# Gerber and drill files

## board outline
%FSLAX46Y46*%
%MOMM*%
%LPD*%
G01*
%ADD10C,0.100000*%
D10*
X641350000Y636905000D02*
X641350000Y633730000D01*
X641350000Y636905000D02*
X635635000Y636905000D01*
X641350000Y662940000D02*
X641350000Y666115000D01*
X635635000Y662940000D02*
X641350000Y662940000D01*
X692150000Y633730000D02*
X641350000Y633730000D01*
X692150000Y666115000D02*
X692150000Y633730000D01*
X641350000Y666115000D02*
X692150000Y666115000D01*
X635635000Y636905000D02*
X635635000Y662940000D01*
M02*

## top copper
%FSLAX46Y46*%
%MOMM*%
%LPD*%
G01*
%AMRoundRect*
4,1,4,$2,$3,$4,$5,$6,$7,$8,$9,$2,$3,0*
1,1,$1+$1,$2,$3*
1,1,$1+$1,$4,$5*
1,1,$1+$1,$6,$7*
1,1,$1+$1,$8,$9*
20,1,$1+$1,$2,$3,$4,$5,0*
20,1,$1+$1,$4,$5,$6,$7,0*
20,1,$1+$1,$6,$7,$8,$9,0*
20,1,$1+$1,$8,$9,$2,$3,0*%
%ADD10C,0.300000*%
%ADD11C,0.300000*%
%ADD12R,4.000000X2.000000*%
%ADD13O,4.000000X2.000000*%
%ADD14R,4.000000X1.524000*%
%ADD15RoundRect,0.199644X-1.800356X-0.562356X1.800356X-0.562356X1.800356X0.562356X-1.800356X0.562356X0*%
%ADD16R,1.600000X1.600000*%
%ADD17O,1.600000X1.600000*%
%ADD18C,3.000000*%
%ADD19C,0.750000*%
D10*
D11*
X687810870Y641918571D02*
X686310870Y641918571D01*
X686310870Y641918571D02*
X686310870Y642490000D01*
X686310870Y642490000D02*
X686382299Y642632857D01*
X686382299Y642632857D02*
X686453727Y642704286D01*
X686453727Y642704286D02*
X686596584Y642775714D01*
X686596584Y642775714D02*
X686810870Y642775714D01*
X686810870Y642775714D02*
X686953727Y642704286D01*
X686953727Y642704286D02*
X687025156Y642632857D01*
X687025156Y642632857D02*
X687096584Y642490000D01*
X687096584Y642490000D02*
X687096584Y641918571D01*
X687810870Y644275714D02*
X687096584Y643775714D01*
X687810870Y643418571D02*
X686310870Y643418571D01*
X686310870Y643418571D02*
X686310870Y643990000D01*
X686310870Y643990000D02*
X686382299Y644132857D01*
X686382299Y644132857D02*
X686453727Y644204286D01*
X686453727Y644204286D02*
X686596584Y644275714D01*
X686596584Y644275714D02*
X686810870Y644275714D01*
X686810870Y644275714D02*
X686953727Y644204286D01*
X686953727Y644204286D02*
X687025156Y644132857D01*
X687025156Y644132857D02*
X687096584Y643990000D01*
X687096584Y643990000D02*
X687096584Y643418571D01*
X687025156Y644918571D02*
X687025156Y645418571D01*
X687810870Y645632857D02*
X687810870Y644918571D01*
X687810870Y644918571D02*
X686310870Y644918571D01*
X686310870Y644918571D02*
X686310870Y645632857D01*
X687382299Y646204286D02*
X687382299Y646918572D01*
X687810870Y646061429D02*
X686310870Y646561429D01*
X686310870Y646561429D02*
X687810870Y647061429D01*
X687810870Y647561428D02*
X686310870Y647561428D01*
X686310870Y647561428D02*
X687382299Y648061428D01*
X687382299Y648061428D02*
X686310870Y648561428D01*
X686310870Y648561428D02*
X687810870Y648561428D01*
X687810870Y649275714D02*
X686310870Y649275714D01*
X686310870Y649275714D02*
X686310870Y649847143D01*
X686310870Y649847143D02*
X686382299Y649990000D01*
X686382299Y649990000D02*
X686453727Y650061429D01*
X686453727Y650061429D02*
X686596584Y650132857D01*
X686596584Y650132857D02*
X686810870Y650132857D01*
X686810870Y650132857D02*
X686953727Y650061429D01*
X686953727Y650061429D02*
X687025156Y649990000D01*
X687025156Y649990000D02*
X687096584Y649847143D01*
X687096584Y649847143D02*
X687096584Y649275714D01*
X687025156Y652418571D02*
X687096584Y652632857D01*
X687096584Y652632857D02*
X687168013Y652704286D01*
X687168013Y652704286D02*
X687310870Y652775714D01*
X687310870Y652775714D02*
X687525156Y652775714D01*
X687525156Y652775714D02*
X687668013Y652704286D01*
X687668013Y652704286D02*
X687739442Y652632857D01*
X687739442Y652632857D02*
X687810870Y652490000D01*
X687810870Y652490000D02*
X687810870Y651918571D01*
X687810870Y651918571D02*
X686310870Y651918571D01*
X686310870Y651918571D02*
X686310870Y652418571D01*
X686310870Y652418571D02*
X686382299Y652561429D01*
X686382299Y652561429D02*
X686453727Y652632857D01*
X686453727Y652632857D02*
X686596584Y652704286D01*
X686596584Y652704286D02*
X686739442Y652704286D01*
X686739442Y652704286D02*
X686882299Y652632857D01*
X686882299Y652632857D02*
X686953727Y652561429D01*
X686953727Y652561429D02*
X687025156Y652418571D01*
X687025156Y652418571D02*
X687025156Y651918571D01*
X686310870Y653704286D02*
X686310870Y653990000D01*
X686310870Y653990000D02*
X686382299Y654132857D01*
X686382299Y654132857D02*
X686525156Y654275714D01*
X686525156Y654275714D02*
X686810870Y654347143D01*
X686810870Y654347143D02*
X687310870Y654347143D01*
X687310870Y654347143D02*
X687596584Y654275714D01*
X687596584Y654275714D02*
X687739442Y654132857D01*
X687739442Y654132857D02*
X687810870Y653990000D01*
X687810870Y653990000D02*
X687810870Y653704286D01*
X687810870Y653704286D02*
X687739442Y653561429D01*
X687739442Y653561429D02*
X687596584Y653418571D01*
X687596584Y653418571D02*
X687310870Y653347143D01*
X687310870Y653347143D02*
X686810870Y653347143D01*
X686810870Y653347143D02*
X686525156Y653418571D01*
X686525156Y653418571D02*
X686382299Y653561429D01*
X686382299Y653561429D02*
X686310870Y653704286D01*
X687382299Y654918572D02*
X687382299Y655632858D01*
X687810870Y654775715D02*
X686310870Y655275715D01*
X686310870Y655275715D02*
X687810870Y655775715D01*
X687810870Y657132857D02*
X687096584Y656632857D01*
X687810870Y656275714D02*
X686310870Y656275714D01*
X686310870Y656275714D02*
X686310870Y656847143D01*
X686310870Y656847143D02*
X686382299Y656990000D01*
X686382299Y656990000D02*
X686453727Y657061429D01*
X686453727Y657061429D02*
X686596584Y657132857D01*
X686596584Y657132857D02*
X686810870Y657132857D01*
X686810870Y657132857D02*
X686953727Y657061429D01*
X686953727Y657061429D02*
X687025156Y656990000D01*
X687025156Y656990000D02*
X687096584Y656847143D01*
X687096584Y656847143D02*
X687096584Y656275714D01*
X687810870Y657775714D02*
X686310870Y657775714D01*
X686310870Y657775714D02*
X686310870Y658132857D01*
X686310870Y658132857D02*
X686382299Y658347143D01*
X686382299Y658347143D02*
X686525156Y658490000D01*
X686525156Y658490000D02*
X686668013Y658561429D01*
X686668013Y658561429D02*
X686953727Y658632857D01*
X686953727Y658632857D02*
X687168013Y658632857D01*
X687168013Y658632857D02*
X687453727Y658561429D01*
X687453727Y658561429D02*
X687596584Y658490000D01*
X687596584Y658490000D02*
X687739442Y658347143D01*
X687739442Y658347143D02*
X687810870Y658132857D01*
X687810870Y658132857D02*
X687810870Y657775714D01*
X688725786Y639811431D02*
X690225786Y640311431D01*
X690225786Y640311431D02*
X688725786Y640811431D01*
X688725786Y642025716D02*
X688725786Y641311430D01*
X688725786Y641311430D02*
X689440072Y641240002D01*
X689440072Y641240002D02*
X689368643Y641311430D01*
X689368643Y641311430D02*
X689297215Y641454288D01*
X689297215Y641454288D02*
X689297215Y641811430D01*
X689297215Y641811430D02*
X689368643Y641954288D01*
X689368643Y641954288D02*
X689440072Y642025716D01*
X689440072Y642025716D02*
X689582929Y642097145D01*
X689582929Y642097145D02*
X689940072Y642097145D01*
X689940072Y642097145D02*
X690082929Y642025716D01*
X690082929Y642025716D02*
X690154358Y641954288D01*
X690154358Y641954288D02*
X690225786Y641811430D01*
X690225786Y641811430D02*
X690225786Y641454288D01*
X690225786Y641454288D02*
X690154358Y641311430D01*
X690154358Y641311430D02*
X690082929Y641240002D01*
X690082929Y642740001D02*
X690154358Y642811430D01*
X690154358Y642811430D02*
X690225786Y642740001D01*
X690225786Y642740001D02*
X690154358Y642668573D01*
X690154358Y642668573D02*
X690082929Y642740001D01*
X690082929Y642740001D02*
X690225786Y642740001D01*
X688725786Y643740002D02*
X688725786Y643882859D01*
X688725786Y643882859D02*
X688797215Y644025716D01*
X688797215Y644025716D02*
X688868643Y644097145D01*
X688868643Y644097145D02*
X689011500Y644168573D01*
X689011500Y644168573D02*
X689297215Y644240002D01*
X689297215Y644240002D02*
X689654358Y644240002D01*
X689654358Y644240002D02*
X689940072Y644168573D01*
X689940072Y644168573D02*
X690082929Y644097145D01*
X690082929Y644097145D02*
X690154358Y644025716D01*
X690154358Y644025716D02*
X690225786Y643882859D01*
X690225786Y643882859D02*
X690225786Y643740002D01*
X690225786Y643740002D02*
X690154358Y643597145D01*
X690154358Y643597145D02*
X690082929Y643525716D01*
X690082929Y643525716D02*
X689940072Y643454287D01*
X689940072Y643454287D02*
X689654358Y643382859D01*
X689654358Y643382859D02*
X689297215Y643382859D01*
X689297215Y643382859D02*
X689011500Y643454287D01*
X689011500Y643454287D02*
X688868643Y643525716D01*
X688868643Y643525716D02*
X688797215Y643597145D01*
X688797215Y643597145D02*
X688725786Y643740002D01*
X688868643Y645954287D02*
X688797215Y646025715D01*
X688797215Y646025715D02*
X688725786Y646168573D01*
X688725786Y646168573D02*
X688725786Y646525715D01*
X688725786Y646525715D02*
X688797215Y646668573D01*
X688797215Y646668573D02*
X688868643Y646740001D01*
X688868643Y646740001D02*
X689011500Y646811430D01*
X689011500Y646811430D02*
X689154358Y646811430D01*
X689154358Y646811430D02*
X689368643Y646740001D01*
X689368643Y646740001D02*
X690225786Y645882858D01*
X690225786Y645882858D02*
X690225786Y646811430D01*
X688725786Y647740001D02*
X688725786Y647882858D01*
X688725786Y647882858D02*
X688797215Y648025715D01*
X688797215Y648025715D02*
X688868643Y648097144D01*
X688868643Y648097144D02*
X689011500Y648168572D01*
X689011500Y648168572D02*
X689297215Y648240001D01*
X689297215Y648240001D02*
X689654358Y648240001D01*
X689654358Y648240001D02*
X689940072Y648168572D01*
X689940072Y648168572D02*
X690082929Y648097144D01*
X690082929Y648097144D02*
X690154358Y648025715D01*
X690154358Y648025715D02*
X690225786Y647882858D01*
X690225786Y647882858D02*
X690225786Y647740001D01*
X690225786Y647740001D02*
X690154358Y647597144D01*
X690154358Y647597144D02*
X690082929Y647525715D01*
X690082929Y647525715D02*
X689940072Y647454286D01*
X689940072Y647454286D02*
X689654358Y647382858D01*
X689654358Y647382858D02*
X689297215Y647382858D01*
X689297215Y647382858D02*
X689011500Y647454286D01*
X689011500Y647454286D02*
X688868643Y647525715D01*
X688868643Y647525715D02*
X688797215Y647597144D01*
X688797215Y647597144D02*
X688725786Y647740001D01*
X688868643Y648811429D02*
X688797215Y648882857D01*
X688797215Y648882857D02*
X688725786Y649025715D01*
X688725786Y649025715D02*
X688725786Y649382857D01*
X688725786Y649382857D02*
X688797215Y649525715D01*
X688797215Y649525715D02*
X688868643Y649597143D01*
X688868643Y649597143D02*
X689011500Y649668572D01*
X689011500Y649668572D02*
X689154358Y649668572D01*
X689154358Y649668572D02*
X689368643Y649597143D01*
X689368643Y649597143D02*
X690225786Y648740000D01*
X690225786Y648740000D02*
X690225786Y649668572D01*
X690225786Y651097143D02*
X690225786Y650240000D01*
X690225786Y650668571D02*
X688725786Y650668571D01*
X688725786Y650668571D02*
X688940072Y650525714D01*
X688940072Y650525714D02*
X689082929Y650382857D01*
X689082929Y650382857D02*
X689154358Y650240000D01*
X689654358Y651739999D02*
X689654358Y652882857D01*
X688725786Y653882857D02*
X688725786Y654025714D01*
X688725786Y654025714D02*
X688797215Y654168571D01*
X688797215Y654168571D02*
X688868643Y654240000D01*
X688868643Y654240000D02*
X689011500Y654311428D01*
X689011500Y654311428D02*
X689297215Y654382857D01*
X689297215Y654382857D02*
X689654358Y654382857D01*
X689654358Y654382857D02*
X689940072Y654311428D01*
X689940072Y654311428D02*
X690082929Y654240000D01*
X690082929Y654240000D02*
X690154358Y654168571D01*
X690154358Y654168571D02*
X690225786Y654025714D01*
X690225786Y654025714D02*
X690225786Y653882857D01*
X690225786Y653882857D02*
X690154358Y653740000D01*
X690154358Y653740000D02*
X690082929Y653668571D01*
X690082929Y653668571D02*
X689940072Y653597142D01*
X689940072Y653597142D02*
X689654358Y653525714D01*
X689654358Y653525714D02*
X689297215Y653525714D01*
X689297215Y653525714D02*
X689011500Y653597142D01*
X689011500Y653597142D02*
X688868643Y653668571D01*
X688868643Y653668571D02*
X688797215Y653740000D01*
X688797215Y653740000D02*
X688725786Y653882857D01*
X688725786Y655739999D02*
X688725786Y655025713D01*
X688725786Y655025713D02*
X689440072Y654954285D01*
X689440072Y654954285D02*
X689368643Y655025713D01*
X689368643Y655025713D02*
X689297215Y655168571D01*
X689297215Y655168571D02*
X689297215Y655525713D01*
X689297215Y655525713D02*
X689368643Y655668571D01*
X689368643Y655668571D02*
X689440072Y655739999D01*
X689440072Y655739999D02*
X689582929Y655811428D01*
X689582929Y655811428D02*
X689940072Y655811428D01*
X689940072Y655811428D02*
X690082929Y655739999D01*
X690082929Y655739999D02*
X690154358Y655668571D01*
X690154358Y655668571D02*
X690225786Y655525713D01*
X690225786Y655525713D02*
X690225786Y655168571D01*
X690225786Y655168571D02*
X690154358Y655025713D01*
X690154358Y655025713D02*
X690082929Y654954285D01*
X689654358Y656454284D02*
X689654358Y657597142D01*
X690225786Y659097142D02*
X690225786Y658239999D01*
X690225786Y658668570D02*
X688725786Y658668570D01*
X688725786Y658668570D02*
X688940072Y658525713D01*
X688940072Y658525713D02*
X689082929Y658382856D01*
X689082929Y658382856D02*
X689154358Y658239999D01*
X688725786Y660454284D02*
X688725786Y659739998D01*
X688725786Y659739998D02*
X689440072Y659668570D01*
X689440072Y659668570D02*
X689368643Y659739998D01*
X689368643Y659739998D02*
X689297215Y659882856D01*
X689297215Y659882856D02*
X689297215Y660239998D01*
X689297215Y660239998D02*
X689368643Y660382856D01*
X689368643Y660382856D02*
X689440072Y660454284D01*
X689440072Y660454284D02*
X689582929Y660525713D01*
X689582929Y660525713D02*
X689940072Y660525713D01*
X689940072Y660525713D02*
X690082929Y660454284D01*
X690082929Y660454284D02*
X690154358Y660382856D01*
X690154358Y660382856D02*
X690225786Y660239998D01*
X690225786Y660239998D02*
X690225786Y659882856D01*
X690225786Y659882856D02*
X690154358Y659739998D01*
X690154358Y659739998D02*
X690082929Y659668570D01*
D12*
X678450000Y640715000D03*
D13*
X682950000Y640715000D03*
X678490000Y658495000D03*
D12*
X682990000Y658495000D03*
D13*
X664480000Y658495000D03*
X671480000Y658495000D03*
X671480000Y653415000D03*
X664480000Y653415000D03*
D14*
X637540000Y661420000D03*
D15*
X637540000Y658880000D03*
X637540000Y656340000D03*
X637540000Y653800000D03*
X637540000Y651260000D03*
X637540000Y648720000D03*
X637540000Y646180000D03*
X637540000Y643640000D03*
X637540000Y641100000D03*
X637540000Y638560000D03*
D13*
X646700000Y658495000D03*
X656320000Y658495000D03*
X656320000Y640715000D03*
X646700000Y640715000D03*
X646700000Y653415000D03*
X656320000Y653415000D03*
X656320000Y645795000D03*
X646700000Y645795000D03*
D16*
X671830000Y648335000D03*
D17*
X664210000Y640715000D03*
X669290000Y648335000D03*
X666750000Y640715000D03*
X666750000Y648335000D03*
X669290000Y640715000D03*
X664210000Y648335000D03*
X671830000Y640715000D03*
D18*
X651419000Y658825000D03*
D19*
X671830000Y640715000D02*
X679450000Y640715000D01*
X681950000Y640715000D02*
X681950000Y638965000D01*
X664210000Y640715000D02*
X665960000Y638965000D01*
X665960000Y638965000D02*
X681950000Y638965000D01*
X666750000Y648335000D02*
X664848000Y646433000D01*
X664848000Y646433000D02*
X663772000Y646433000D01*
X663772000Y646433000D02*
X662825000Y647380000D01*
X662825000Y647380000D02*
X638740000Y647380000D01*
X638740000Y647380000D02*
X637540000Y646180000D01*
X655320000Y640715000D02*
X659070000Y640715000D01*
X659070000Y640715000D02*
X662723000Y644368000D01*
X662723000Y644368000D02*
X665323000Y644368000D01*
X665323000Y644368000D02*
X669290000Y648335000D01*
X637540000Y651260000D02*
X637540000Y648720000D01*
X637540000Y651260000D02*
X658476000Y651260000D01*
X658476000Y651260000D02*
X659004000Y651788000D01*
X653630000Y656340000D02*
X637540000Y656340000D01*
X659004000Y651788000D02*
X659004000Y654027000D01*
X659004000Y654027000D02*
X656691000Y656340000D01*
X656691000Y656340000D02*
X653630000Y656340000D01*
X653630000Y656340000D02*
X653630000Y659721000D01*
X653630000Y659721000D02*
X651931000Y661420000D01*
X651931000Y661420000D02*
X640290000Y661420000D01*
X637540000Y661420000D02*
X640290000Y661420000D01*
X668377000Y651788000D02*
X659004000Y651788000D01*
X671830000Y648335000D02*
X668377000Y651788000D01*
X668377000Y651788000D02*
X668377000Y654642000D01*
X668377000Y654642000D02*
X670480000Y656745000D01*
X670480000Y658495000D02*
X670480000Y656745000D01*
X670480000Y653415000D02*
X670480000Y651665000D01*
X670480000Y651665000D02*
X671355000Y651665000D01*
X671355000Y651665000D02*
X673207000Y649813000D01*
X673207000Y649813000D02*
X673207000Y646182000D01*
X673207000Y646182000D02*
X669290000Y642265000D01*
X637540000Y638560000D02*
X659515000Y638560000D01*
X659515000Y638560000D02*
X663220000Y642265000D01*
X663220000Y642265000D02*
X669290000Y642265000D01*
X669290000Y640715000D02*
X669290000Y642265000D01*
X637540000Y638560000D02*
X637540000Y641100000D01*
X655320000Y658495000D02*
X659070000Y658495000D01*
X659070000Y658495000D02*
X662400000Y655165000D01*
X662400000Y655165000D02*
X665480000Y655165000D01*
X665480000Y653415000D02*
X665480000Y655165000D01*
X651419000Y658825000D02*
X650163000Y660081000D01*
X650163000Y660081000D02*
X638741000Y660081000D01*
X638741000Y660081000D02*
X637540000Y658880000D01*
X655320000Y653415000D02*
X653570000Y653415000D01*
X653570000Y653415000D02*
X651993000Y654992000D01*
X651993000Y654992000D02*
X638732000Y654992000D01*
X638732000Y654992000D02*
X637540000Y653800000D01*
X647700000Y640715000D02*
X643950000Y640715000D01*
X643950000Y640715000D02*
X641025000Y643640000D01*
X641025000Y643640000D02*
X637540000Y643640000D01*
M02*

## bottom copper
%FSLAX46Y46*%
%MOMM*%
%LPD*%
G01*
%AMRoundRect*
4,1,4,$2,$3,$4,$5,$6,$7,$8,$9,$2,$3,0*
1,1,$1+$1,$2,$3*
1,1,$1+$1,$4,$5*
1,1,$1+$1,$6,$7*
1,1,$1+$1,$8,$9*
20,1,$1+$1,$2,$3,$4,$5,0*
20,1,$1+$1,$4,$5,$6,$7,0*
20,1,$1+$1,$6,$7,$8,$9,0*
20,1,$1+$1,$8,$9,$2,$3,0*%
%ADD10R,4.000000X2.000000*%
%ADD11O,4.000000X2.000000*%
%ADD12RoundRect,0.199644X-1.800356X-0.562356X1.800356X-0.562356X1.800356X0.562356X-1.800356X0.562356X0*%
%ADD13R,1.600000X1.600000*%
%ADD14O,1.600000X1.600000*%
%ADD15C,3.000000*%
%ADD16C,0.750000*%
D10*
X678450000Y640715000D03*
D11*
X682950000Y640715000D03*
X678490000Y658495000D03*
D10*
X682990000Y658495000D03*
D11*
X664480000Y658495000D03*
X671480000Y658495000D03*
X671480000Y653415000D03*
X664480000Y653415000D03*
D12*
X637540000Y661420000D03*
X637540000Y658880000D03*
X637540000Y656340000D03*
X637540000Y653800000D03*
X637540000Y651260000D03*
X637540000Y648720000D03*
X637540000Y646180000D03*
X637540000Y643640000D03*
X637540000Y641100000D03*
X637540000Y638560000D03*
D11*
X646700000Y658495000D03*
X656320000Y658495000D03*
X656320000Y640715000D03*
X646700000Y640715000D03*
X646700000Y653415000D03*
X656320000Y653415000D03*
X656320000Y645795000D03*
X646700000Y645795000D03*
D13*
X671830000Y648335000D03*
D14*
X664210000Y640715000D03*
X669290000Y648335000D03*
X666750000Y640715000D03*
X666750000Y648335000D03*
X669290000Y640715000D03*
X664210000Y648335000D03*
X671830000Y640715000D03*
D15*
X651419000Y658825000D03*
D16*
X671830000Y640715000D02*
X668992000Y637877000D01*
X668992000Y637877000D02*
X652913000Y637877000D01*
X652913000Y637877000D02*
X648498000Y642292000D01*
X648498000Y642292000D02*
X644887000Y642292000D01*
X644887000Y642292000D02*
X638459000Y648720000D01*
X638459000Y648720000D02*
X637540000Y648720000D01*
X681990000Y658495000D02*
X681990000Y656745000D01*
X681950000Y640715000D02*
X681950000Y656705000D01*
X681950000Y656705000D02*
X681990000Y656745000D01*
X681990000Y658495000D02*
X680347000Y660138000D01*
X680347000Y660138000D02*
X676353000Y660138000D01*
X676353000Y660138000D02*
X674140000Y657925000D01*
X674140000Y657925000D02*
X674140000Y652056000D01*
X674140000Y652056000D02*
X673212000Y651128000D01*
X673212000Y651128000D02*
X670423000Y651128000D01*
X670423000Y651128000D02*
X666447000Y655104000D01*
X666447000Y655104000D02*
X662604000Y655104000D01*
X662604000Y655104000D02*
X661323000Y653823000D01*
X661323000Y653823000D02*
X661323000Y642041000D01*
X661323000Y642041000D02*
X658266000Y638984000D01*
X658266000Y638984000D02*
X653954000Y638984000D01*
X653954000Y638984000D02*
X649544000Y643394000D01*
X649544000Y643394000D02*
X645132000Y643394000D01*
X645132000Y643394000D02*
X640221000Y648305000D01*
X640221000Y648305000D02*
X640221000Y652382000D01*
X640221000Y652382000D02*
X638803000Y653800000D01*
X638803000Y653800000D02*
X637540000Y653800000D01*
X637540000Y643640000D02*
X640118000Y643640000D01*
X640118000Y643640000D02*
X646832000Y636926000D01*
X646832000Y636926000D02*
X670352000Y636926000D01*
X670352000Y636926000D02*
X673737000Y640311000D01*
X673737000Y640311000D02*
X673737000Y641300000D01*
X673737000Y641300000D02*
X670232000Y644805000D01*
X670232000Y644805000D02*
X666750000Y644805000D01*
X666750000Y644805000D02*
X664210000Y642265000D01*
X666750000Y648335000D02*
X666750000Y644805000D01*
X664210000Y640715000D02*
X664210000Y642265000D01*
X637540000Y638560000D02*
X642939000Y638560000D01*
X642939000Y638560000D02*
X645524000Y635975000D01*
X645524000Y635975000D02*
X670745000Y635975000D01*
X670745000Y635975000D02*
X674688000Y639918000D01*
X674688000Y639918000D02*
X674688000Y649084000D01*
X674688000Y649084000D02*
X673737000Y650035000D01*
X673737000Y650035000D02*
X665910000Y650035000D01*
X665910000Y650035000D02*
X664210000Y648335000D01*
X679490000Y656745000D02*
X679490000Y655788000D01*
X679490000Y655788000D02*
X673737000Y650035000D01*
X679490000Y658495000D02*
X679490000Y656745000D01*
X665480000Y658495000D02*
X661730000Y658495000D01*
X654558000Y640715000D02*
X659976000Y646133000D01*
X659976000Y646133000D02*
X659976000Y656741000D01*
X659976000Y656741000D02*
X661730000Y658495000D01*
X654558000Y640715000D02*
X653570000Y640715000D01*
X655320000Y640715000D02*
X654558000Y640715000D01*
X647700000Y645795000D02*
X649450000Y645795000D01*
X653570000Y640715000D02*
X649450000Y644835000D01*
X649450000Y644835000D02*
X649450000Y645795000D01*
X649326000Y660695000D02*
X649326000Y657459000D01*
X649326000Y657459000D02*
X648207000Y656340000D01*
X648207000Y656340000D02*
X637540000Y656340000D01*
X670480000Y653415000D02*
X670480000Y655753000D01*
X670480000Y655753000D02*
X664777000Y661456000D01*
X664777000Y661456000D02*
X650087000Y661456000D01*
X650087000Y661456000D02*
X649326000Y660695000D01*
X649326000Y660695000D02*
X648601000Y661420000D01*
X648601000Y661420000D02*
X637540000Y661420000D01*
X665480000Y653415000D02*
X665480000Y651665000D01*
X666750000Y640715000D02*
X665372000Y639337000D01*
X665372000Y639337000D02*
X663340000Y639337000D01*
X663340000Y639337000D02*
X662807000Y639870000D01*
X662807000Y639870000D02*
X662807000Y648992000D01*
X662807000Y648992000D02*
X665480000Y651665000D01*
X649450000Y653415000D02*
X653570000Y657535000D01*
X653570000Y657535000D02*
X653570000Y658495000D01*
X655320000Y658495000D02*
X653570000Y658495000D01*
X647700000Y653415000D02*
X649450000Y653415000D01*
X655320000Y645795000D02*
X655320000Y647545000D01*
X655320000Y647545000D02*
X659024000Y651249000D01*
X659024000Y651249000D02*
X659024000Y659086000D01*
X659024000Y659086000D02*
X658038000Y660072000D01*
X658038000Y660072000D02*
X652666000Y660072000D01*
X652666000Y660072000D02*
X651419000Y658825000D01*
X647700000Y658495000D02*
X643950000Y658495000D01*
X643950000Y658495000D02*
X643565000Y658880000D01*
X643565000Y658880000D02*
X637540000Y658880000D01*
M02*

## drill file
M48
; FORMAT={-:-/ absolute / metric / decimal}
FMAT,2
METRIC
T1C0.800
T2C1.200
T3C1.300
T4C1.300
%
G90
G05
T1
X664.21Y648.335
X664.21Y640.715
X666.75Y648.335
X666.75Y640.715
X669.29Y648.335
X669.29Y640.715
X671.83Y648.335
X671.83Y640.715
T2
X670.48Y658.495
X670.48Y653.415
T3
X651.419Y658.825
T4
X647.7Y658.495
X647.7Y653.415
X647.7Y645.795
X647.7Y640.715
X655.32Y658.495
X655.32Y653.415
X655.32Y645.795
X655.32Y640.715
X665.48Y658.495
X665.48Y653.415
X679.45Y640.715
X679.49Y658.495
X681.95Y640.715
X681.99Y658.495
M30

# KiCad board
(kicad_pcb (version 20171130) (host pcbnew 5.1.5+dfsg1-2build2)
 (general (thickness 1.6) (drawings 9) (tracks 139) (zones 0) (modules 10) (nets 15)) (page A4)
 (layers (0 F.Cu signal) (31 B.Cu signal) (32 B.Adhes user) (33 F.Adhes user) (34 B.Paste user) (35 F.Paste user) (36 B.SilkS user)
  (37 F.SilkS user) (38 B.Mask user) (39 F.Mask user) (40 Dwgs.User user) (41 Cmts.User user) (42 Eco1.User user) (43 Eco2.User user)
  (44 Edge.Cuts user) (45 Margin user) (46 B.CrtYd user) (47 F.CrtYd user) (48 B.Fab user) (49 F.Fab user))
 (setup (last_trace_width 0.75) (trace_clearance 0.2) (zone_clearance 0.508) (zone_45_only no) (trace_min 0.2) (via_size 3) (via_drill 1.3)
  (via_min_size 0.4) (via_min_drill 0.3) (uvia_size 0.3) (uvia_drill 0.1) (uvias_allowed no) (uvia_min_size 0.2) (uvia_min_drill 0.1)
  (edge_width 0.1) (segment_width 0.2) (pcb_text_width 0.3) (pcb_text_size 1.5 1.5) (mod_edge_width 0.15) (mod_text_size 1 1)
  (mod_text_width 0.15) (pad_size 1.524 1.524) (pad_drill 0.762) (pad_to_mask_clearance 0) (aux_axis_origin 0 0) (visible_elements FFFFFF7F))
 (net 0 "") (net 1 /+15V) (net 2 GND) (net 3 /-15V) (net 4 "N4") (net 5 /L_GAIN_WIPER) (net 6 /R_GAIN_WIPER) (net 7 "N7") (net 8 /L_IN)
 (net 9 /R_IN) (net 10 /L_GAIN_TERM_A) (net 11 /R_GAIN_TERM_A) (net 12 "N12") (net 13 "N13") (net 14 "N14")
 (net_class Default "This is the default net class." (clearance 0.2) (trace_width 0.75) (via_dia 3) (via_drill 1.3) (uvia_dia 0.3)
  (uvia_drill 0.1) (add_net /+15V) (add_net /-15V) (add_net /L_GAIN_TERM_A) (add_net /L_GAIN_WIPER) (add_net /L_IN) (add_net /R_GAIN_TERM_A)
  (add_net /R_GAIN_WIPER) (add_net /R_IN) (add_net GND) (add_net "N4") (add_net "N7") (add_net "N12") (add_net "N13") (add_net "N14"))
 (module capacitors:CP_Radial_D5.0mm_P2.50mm (layer F.Cu) (at 679.45 -640.715)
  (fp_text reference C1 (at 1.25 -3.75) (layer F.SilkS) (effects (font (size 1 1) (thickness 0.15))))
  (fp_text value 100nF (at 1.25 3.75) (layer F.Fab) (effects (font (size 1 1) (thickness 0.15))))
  (pad 1 thru_hole rect (at 0 0) (size 4 2) (drill 1.3 (offset -1 0)) (layers *.Cu *.Mask) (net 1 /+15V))
  (pad 2 thru_hole oval (at 2.5 0) (size 4 2) (drill 1.3 (offset 1 0)) (layers *.Cu *.Mask) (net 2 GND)))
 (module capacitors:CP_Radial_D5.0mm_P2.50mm (layer F.Cu) (at 681.99 -658.495 180)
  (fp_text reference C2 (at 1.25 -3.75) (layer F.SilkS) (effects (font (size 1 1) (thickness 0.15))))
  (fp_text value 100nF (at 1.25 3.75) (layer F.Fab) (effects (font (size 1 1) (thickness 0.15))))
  (pad 2 thru_hole oval (at 2.5 0 180) (size 4 2) (drill 1.3 (offset 1 0)) (layers *.Cu *.Mask) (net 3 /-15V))
  (pad 1 thru_hole rect (at 0 0 180) (size 4 2) (drill 1.3 (offset -1 0)) (layers *.Cu *.Mask) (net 2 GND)))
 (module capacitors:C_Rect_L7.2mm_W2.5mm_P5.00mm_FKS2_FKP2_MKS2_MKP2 (layer F.Cu) (at 665.48 -658.495)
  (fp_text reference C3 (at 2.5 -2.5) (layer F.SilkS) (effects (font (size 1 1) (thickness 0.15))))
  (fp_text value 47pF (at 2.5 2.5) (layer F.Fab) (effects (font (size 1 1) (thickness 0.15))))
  (pad 1 thru_hole oval (at 0 0) (size 4 2) (drill 1.3 (offset -1 0)) (layers *.Cu *.Mask) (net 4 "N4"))
  (pad 2 thru_hole oval (at 5 0) (size 4 2) (drill 1.2 (offset 1 0)) (layers *.Cu *.Mask) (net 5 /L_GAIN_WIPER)))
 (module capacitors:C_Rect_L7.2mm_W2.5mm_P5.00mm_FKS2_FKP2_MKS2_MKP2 (layer F.Cu) (at 665.48 -653.415)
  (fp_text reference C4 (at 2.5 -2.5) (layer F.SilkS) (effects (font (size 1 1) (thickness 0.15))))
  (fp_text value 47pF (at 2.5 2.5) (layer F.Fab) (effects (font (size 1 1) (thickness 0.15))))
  (pad 2 thru_hole oval (at 5 0) (size 4 2) (drill 1.2 (offset 1 0)) (layers *.Cu *.Mask) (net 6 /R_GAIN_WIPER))
  (pad 1 thru_hole oval (at 0 0) (size 4 2) (drill 1.3 (offset -1 0)) (layers *.Cu *.Mask) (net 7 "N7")))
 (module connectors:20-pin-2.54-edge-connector (layer F.Cu) (at 645.16 -663.96)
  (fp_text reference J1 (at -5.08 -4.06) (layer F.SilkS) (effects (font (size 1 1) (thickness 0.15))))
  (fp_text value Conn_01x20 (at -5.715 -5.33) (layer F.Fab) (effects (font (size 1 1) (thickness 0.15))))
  (pad 1 connect rect (at -7.62 2.54) (size 4 1.524) (layers F.Cu F.Mask) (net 5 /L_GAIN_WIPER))
  (pad 2 connect roundrect (at -7.62 5.08) (size 4 1.524) (layers F.Cu F.Mask) (roundrect_rratio 0.131) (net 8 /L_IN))
  (pad 3 connect roundrect (at -7.62 7.62) (size 4 1.524) (layers F.Cu F.Mask) (roundrect_rratio 0.131) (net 5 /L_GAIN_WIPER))
  (pad 4 connect roundrect (at -7.62 10.16) (size 4 1.524) (layers F.Cu F.Mask) (roundrect_rratio 0.131) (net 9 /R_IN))
  (pad 5 connect roundrect (at -7.62 12.7) (size 4 1.524) (layers F.Cu F.Mask) (roundrect_rratio 0.131) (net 5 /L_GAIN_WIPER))
  (pad 6 connect roundrect (at -7.62 15.24) (size 4 1.524) (layers F.Cu F.Mask) (roundrect_rratio 0.131) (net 5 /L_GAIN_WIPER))
  (pad 7 connect roundrect (at -7.62 17.78) (size 4 1.524) (layers F.Cu F.Mask) (roundrect_rratio 0.131) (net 2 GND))
  (pad 8 connect roundrect (at -7.62 20.32) (size 4 1.524) (layers F.Cu F.Mask) (roundrect_rratio 0.131) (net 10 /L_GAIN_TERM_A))
  (pad 9 connect roundrect (at -7.62 22.86) (size 4 1.524) (layers F.Cu F.Mask) (roundrect_rratio 0.131) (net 6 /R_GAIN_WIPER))
  (pad 10 connect roundrect (at -7.62 25.4) (size 4 1.524) (layers F.Cu F.Mask) (roundrect_rratio 0.131) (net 6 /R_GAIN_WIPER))
  (pad 11 connect roundrect (at -7.62 2.54) (size 4 1.524) (layers B.Cu B.Mask) (roundrect_rratio 0.131) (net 6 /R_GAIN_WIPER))
  (pad 12 connect roundrect (at -7.62 5.08) (size 4 1.524) (layers B.Cu B.Mask) (roundrect_rratio 0.131) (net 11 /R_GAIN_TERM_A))
  (pad 13 connect roundrect (at -7.62 7.62) (size 4 1.524) (layers B.Cu B.Mask) (roundrect_rratio 0.131) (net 6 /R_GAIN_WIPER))
  (pad 14 connect roundrect (at -7.62 10.16) (size 4 1.524) (layers B.Cu B.Mask) (roundrect_rratio 0.131) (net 2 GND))
  (pad 15 connect roundrect (at -7.62 12.7) (size 4 1.524) (layers B.Cu B.Mask) (roundrect_rratio 0.131) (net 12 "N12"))
  (pad 16 connect roundrect (at -7.62 15.24) (size 4 1.524) (layers B.Cu B.Mask) (roundrect_rratio 0.131) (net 1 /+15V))
  (pad 17 connect roundrect (at -7.62 17.78) (size 4 1.524) (layers B.Cu B.Mask) (roundrect_rratio 0.131) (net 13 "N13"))
  (pad 18 connect roundrect (at -7.62 20.32) (size 4 1.524) (layers B.Cu B.Mask) (roundrect_rratio 0.131) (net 2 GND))
  (pad 19 connect roundrect (at -7.62 22.86) (size 4 1.524) (layers B.Cu B.Mask) (roundrect_rratio 0.131) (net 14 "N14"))
  (pad 20 connect roundrect (at -7.62 25.4) (size 4 1.524) (layers B.Cu B.Mask) (roundrect_rratio 0.131) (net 3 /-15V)))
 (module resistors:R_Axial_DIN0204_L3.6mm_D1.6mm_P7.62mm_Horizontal (layer F.Cu) (at 655.32 -658.495 180)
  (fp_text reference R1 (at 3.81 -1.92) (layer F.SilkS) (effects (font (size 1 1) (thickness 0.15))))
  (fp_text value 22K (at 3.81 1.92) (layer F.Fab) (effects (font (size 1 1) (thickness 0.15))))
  (pad 2 thru_hole oval (at 7.62 0 180) (size 4 2) (drill 1.3 (offset 1 0)) (layers *.Cu *.Mask) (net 11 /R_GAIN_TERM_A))
  (pad 1 thru_hole oval (at 0 0 180) (size 4 2) (drill 1.3 (offset -1 0)) (layers *.Cu *.Mask) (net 7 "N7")))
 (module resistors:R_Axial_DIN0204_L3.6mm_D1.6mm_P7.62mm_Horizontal (layer F.Cu) (at 655.32 -640.715 180)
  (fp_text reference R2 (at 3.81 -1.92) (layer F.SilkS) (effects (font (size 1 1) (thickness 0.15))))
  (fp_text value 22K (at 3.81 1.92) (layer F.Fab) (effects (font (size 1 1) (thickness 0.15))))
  (pad 1 thru_hole oval (at 0 0 180) (size 4 2) (drill 1.3 (offset -1 0)) (layers *.Cu *.Mask) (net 4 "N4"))
  (pad 2 thru_hole oval (at 7.62 0 180) (size 4 2) (drill 1.3 (offset 1 0)) (layers *.Cu *.Mask) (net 10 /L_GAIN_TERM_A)))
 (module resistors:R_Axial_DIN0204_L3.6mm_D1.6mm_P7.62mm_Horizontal (layer F.Cu) (at 647.7 -653.415)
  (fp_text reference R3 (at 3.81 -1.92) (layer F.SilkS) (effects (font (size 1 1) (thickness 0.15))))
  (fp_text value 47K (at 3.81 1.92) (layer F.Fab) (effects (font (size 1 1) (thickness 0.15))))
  (pad 1 thru_hole oval (at 0 0) (size 4 2) (drill 1.3 (offset -1 0)) (layers *.Cu *.Mask) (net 7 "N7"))
  (pad 2 thru_hole oval (at 7.62 0) (size 4 2) (drill 1.3 (offset 1 0)) (layers *.Cu *.Mask) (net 9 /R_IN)))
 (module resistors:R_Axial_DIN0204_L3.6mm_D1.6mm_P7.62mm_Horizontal (layer F.Cu) (at 647.7 -645.795)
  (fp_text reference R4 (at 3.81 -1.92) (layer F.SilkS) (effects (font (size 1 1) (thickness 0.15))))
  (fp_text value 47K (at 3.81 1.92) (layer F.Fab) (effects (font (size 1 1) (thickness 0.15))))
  (pad 2 thru_hole oval (at 7.62 0) (size 4 2) (drill 1.3 (offset 1 0)) (layers *.Cu *.Mask) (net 8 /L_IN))
  (pad 1 thru_hole oval (at 0 0) (size 4 2) (drill 1.3 (offset -1 0)) (layers *.Cu *.Mask) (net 4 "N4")))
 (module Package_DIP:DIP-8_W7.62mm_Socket (layer F.Cu) (at 671.83 -648.335 270)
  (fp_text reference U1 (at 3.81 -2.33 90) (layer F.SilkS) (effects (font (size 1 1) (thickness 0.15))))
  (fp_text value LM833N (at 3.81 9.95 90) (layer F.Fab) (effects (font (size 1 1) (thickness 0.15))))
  (pad 1 thru_hole rect (at 0 0 270) (size 1.6 1.6) (drill 0.8) (layers *.Cu *.Mask) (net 5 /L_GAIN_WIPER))
  (pad 5 thru_hole oval (at 7.62 7.62 270) (size 1.6 1.6) (drill 0.8) (layers *.Cu *.Mask) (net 2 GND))
  (pad 2 thru_hole oval (at 0 2.54 270) (size 1.6 1.6) (drill 0.8) (layers *.Cu *.Mask) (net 4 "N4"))
  (pad 6 thru_hole oval (at 7.62 5.08 270) (size 1.6 1.6) (drill 0.8) (layers *.Cu *.Mask) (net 7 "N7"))
  (pad 3 thru_hole oval (at 0 5.08 270) (size 1.6 1.6) (drill 0.8) (layers *.Cu *.Mask) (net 2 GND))
  (pad 7 thru_hole oval (at 7.62 2.54 270) (size 1.6 1.6) (drill 0.8) (layers *.Cu *.Mask) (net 6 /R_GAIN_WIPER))
  (pad 4 thru_hole oval (at 0 7.62 270) (size 1.6 1.6) (drill 0.8) (layers *.Cu *.Mask) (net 3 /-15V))
  (pad 8 thru_hole oval (at 7.62 0 270) (size 1.6 1.6) (drill 0.8) (layers *.Cu *.Mask) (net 1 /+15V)))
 (gr_line (start 641.35 -636.905) (end 641.35 -633.73) (layer Edge.Cuts) (width 0.1))
 (gr_line (start 641.35 -636.905) (end 635.635 -636.905) (layer Edge.Cuts) (width 0.1))
 (gr_line (start 641.35 -662.94) (end 641.35 -666.115) (layer Edge.Cuts) (width 0.1))
 (gr_line (start 635.635 -662.94) (end 641.35 -662.94) (layer Edge.Cuts) (width 0.1))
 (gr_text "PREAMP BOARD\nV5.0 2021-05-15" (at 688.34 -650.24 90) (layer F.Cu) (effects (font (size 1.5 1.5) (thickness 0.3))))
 (gr_line (start 692.15 -633.73) (end 641.35 -633.73) (layer Edge.Cuts) (width 0.1))
 (gr_line (start 692.15 -666.115) (end 692.15 -633.73) (layer Edge.Cuts) (width 0.1))
 (gr_line (start 641.35 -666.115) (end 692.15 -666.115) (layer Edge.Cuts) (width 0.1))
 (gr_line (start 635.635 -636.905) (end 635.635 -662.94) (layer Edge.Cuts) (width 0.1))
 (segment (start 671.83 -640.715) (end 668.992 -637.877) (width 0.75) (layer B.Cu) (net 1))
 (segment (start 668.992 -637.877) (end 652.913 -637.877) (width 0.75) (layer B.Cu) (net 1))
 (segment (start 652.913 -637.877) (end 648.498 -642.292) (width 0.75) (layer B.Cu) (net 1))
 (segment (start 648.498 -642.292) (end 644.887 -642.292) (width 0.75) (layer B.Cu) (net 1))
 (segment (start 644.887 -642.292) (end 638.459 -648.72) (width 0.75) (layer B.Cu) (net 1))
 (segment (start 638.459 -648.72) (end 637.54 -648.72) (width 0.75) (layer B.Cu) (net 1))
 (segment (start 671.83 -640.715) (end 679.45 -640.715) (width 0.75) (layer F.Cu) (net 1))
 (segment (start 681.99 -658.495) (end 681.99 -656.745) (width 0.75) (layer B.Cu) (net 2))
 (segment (start 681.95 -640.715) (end 681.95 -656.705) (width 0.75) (layer B.Cu) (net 2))
 (segment (start 681.95 -656.705) (end 681.99 -656.745) (width 0.75) (layer B.Cu) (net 2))
 (segment (start 681.99 -658.495) (end 680.347 -660.138) (width 0.75) (layer B.Cu) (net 2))
 (segment (start 680.347 -660.138) (end 676.353 -660.138) (width 0.75) (layer B.Cu) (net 2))
 (segment (start 676.353 -660.138) (end 674.14 -657.925) (width 0.75) (layer B.Cu) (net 2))
 (segment (start 674.14 -657.925) (end 674.14 -652.056) (width 0.75) (layer B.Cu) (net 2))
 (segment (start 674.14 -652.056) (end 673.212 -651.128) (width 0.75) (layer B.Cu) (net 2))
 (segment (start 673.212 -651.128) (end 670.423 -651.128) (width 0.75) (layer B.Cu) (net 2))
 (segment (start 670.423 -651.128) (end 666.447 -655.104) (width 0.75) (layer B.Cu) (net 2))
 (segment (start 666.447 -655.104) (end 662.604 -655.104) (width 0.75) (layer B.Cu) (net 2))
 (segment (start 662.604 -655.104) (end 661.323 -653.823) (width 0.75) (layer B.Cu) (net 2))
 (segment (start 661.323 -653.823) (end 661.323 -642.041) (width 0.75) (layer B.Cu) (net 2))
 (segment (start 661.323 -642.041) (end 658.266 -638.984) (width 0.75) (layer B.Cu) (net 2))
 (segment (start 658.266 -638.984) (end 653.954 -638.984) (width 0.75) (layer B.Cu) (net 2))
 (segment (start 653.954 -638.984) (end 649.544 -643.394) (width 0.75) (layer B.Cu) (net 2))
 (segment (start 649.544 -643.394) (end 645.132 -643.394) (width 0.75) (layer B.Cu) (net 2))
 (segment (start 645.132 -643.394) (end 640.221 -648.305) (width 0.75) (layer B.Cu) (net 2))
 (segment (start 640.221 -648.305) (end 640.221 -652.382) (width 0.75) (layer B.Cu) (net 2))
 (segment (start 640.221 -652.382) (end 638.803 -653.8) (width 0.75) (layer B.Cu) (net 2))
 (segment (start 638.803 -653.8) (end 637.54 -653.8) (width 0.75) (layer B.Cu) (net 2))
 (segment (start 637.54 -643.64) (end 640.118 -643.64) (width 0.75) (layer B.Cu) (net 2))
 (segment (start 640.118 -643.64) (end 646.832 -636.926) (width 0.75) (layer B.Cu) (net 2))
 (segment (start 646.832 -636.926) (end 670.352 -636.926) (width 0.75) (layer B.Cu) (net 2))
 (segment (start 670.352 -636.926) (end 673.737 -640.311) (width 0.75) (layer B.Cu) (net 2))
 (segment (start 673.737 -640.311) (end 673.737 -641.3) (width 0.75) (layer B.Cu) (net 2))
 (segment (start 673.737 -641.3) (end 670.232 -644.805) (width 0.75) (layer B.Cu) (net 2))
 (segment (start 670.232 -644.805) (end 666.75 -644.805) (width 0.75) (layer B.Cu) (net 2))
 (segment (start 681.95 -640.715) (end 681.95 -638.965) (width 0.75) (layer F.Cu) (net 2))
 (segment (start 664.21 -640.715) (end 665.96 -638.965) (width 0.75) (layer F.Cu) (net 2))
 (segment (start 665.96 -638.965) (end 681.95 -638.965) (width 0.75) (layer F.Cu) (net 2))
 (segment (start 666.75 -644.805) (end 664.21 -642.265) (width 0.75) (layer B.Cu) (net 2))
 (segment (start 666.75 -648.335) (end 664.848 -646.433) (width 0.75) (layer F.Cu) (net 2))
 (segment (start 664.848 -646.433) (end 663.772 -646.433) (width 0.75) (layer F.Cu) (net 2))
 (segment (start 663.772 -646.433) (end 662.825 -647.38) (width 0.75) (layer F.Cu) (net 2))
 (segment (start 662.825 -647.38) (end 638.74 -647.38) (width 0.75) (layer F.Cu) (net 2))
 (segment (start 638.74 -647.38) (end 637.54 -646.18) (width 0.75) (layer F.Cu) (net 2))
 (segment (start 666.75 -648.335) (end 666.75 -644.805) (width 0.75) (layer B.Cu) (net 2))
 (segment (start 664.21 -640.715) (end 664.21 -642.265) (width 0.75) (layer B.Cu) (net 2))
 (segment (start 637.54 -638.56) (end 642.939 -638.56) (width 0.75) (layer B.Cu) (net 3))
 (segment (start 642.939 -638.56) (end 645.524 -635.975) (width 0.75) (layer B.Cu) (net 3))
 (segment (start 645.524 -635.975) (end 670.745 -635.975) (width 0.75) (layer B.Cu) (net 3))
 (segment (start 670.745 -635.975) (end 674.688 -639.918) (width 0.75) (layer B.Cu) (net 3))
 (segment (start 674.688 -639.918) (end 674.688 -649.084) (width 0.75) (layer B.Cu) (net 3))
 (segment (start 674.688 -649.084) (end 673.737 -650.035) (width 0.75) (layer B.Cu) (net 3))
 (segment (start 673.737 -650.035) (end 665.91 -650.035) (width 0.75) (layer B.Cu) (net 3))
 (segment (start 665.91 -650.035) (end 664.21 -648.335) (width 0.75) (layer B.Cu) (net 3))
 (segment (start 679.49 -656.745) (end 679.49 -655.788) (width 0.75) (layer B.Cu) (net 3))
 (segment (start 679.49 -655.788) (end 673.737 -650.035) (width 0.75) (layer B.Cu) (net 3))
 (segment (start 679.49 -658.495) (end 679.49 -656.745) (width 0.75) (layer B.Cu) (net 3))
 (segment (start 665.48 -658.495) (end 661.73 -658.495) (width 0.75) (layer B.Cu) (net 4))
 (segment (start 654.558 -640.715) (end 659.976 -646.133) (width 0.75) (layer B.Cu) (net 4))
 (segment (start 659.976 -646.133) (end 659.976 -656.741) (width 0.75) (layer B.Cu) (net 4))
 (segment (start 659.976 -656.741) (end 661.73 -658.495) (width 0.75) (layer B.Cu) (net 4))
 (segment (start 654.558 -640.715) (end 653.57 -640.715) (width 0.75) (layer B.Cu) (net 4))
 (segment (start 655.32 -640.715) (end 654.558 -640.715) (width 0.75) (layer B.Cu) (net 4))
 (segment (start 647.7 -645.795) (end 649.45 -645.795) (width 0.75) (layer B.Cu) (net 4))
 (segment (start 653.57 -640.715) (end 649.45 -644.835) (width 0.75) (layer B.Cu) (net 4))
 (segment (start 649.45 -644.835) (end 649.45 -645.795) (width 0.75) (layer B.Cu) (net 4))
 (segment (start 655.32 -640.715) (end 659.07 -640.715) (width 0.75) (layer F.Cu) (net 4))
 (segment (start 659.07 -640.715) (end 662.723 -644.368) (width 0.75) (layer F.Cu) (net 4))
 (segment (start 662.723 -644.368) (end 665.323 -644.368) (width 0.75) (layer F.Cu) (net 4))
 (segment (start 665.323 -644.368) (end 669.29 -648.335) (width 0.75) (layer F.Cu) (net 4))
 (segment (start 637.54 -651.26) (end 637.54 -648.72) (width 0.75) (layer F.Cu) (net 5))
 (segment (start 637.54 -651.26) (end 658.476 -651.26) (width 0.75) (layer F.Cu) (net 5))
 (segment (start 658.476 -651.26) (end 659.004 -651.788) (width 0.75) (layer F.Cu) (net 5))
 (segment (start 653.63 -656.34) (end 637.54 -656.34) (width 0.75) (layer F.Cu) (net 5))
 (segment (start 659.004 -651.788) (end 659.004 -654.027) (width 0.75) (layer F.Cu) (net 5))
 (segment (start 659.004 -654.027) (end 656.691 -656.34) (width 0.75) (layer F.Cu) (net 5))
 (segment (start 656.691 -656.34) (end 653.63 -656.34) (width 0.75) (layer F.Cu) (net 5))
 (segment (start 653.63 -656.34) (end 653.63 -659.721) (width 0.75) (layer F.Cu) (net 5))
 (segment (start 653.63 -659.721) (end 651.931 -661.42) (width 0.75) (layer F.Cu) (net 5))
 (segment (start 651.931 -661.42) (end 640.29 -661.42) (width 0.75) (layer F.Cu) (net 5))
 (segment (start 637.54 -661.42) (end 640.29 -661.42) (width 0.75) (layer F.Cu) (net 5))
 (segment (start 668.377 -651.788) (end 659.004 -651.788) (width 0.75) (layer F.Cu) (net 5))
 (segment (start 671.83 -648.335) (end 668.377 -651.788) (width 0.75) (layer F.Cu) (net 5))
 (segment (start 668.377 -651.788) (end 668.377 -654.642) (width 0.75) (layer F.Cu) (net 5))
 (segment (start 668.377 -654.642) (end 670.48 -656.745) (width 0.75) (layer F.Cu) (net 5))
 (segment (start 670.48 -658.495) (end 670.48 -656.745) (width 0.75) (layer F.Cu) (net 5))
 (segment (start 649.326 -660.695) (end 649.326 -657.459) (width 0.75) (layer B.Cu) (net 6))
 (segment (start 649.326 -657.459) (end 648.207 -656.34) (width 0.75) (layer B.Cu) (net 6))
 (segment (start 648.207 -656.34) (end 637.54 -656.34) (width 0.75) (layer B.Cu) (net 6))
 (segment (start 670.48 -653.415) (end 670.48 -655.753) (width 0.75) (layer B.Cu) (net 6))
 (segment (start 670.48 -655.753) (end 664.777 -661.456) (width 0.75) (layer B.Cu) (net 6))
 (segment (start 664.777 -661.456) (end 650.087 -661.456) (width 0.75) (layer B.Cu) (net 6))
 (segment (start 650.087 -661.456) (end 649.326 -660.695) (width 0.75) (layer B.Cu) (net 6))
 (segment (start 649.326 -660.695) (end 648.601 -661.42) (width 0.75) (layer B.Cu) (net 6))
 (segment (start 648.601 -661.42) (end 637.54 -661.42) (width 0.75) (layer B.Cu) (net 6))
 (segment (start 670.48 -653.415) (end 670.48 -651.665) (width 0.75) (layer F.Cu) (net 6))
 (segment (start 670.48 -651.665) (end 671.355 -651.665) (width 0.75) (layer F.Cu) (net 6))
 (segment (start 671.355 -651.665) (end 673.207 -649.813) (width 0.75) (layer F.Cu) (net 6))
 (segment (start 673.207 -649.813) (end 673.207 -646.182) (width 0.75) (layer F.Cu) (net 6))
 (segment (start 673.207 -646.182) (end 669.29 -642.265) (width 0.75) (layer F.Cu) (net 6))
 (segment (start 637.54 -638.56) (end 659.515 -638.56) (width 0.75) (layer F.Cu) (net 6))
 (segment (start 659.515 -638.56) (end 663.22 -642.265) (width 0.75) (layer F.Cu) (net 6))
 (segment (start 663.22 -642.265) (end 669.29 -642.265) (width 0.75) (layer F.Cu) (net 6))
 (segment (start 669.29 -640.715) (end 669.29 -642.265) (width 0.75) (layer F.Cu) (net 6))
 (segment (start 637.54 -638.56) (end 637.54 -641.1) (width 0.75) (layer F.Cu) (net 6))
 (segment (start 665.48 -653.415) (end 665.48 -651.665) (width 0.75) (layer B.Cu) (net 7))
 (segment (start 666.75 -640.715) (end 665.372 -639.337) (width 0.75) (layer B.Cu) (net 7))
 (segment (start 665.372 -639.337) (end 663.34 -639.337) (width 0.75) (layer B.Cu) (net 7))
 (segment (start 663.34 -639.337) (end 662.807 -639.87) (width 0.75) (layer B.Cu) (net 7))
 (segment (start 662.807 -639.87) (end 662.807 -648.992) (width 0.75) (layer B.Cu) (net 7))
 (segment (start 662.807 -648.992) (end 665.48 -651.665) (width 0.75) (layer B.Cu) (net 7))
 (segment (start 655.32 -658.495) (end 659.07 -658.495) (width 0.75) (layer F.Cu) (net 7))
 (segment (start 659.07 -658.495) (end 662.4 -655.165) (width 0.75) (layer F.Cu) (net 7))
 (segment (start 662.4 -655.165) (end 665.48 -655.165) (width 0.75) (layer F.Cu) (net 7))
 (segment (start 665.48 -653.415) (end 665.48 -655.165) (width 0.75) (layer F.Cu) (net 7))
 (segment (start 649.45 -653.415) (end 653.57 -657.535) (width 0.75) (layer B.Cu) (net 7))
 (segment (start 653.57 -657.535) (end 653.57 -658.495) (width 0.75) (layer B.Cu) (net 7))
 (segment (start 655.32 -658.495) (end 653.57 -658.495) (width 0.75) (layer B.Cu) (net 7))
 (segment (start 647.7 -653.415) (end 649.45 -653.415) (width 0.75) (layer B.Cu) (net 7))
 (segment (start 655.32 -645.795) (end 655.32 -647.545) (width 0.75) (layer B.Cu) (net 8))
 (segment (start 651.419 -658.825) (end 650.163 -660.081) (width 0.75) (layer F.Cu) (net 8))
 (segment (start 650.163 -660.081) (end 638.741 -660.081) (width 0.75) (layer F.Cu) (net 8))
 (segment (start 638.741 -660.081) (end 637.54 -658.88) (width 0.75) (layer F.Cu) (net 8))
 (segment (start 655.32 -647.545) (end 659.024 -651.249) (width 0.75) (layer B.Cu) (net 8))
 (segment (start 659.024 -651.249) (end 659.024 -659.086) (width 0.75) (layer B.Cu) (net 8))
 (segment (start 659.024 -659.086) (end 658.038 -660.072) (width 0.75) (layer B.Cu) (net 8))
 (segment (start 658.038 -660.072) (end 652.666 -660.072) (width 0.75) (layer B.Cu) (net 8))
 (segment (start 652.666 -660.072) (end 651.419 -658.825) (width 0.75) (layer B.Cu) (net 8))
 (via (at 651.419 -658.825) (size 3) (layers F.Cu B.Cu) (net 8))
 (segment (start 655.32 -653.415) (end 653.57 -653.415) (width 0.75) (layer F.Cu) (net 9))
 (segment (start 653.57 -653.415) (end 651.993 -654.992) (width 0.75) (layer F.Cu) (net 9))
 (segment (start 651.993 -654.992) (end 638.732 -654.992) (width 0.75) (layer F.Cu) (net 9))
 (segment (start 638.732 -654.992) (end 637.54 -653.8) (width 0.75) (layer F.Cu) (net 9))
 (segment (start 647.7 -640.715) (end 643.95 -640.715) (width 0.75) (layer F.Cu) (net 10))
 (segment (start 643.95 -640.715) (end 641.025 -643.64) (width 0.75) (layer F.Cu) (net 10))
 (segment (start 641.025 -643.64) (end 637.54 -643.64) (width 0.75) (layer F.Cu) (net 10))
 (segment (start 647.7 -658.495) (end 643.95 -658.495) (width 0.75) (layer B.Cu) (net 11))
 (segment (start 643.95 -658.495) (end 643.565 -658.88) (width 0.75) (layer B.Cu) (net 11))
 (segment (start 643.565 -658.88) (end 637.54 -658.88) (width 0.75) (layer B.Cu) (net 11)))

